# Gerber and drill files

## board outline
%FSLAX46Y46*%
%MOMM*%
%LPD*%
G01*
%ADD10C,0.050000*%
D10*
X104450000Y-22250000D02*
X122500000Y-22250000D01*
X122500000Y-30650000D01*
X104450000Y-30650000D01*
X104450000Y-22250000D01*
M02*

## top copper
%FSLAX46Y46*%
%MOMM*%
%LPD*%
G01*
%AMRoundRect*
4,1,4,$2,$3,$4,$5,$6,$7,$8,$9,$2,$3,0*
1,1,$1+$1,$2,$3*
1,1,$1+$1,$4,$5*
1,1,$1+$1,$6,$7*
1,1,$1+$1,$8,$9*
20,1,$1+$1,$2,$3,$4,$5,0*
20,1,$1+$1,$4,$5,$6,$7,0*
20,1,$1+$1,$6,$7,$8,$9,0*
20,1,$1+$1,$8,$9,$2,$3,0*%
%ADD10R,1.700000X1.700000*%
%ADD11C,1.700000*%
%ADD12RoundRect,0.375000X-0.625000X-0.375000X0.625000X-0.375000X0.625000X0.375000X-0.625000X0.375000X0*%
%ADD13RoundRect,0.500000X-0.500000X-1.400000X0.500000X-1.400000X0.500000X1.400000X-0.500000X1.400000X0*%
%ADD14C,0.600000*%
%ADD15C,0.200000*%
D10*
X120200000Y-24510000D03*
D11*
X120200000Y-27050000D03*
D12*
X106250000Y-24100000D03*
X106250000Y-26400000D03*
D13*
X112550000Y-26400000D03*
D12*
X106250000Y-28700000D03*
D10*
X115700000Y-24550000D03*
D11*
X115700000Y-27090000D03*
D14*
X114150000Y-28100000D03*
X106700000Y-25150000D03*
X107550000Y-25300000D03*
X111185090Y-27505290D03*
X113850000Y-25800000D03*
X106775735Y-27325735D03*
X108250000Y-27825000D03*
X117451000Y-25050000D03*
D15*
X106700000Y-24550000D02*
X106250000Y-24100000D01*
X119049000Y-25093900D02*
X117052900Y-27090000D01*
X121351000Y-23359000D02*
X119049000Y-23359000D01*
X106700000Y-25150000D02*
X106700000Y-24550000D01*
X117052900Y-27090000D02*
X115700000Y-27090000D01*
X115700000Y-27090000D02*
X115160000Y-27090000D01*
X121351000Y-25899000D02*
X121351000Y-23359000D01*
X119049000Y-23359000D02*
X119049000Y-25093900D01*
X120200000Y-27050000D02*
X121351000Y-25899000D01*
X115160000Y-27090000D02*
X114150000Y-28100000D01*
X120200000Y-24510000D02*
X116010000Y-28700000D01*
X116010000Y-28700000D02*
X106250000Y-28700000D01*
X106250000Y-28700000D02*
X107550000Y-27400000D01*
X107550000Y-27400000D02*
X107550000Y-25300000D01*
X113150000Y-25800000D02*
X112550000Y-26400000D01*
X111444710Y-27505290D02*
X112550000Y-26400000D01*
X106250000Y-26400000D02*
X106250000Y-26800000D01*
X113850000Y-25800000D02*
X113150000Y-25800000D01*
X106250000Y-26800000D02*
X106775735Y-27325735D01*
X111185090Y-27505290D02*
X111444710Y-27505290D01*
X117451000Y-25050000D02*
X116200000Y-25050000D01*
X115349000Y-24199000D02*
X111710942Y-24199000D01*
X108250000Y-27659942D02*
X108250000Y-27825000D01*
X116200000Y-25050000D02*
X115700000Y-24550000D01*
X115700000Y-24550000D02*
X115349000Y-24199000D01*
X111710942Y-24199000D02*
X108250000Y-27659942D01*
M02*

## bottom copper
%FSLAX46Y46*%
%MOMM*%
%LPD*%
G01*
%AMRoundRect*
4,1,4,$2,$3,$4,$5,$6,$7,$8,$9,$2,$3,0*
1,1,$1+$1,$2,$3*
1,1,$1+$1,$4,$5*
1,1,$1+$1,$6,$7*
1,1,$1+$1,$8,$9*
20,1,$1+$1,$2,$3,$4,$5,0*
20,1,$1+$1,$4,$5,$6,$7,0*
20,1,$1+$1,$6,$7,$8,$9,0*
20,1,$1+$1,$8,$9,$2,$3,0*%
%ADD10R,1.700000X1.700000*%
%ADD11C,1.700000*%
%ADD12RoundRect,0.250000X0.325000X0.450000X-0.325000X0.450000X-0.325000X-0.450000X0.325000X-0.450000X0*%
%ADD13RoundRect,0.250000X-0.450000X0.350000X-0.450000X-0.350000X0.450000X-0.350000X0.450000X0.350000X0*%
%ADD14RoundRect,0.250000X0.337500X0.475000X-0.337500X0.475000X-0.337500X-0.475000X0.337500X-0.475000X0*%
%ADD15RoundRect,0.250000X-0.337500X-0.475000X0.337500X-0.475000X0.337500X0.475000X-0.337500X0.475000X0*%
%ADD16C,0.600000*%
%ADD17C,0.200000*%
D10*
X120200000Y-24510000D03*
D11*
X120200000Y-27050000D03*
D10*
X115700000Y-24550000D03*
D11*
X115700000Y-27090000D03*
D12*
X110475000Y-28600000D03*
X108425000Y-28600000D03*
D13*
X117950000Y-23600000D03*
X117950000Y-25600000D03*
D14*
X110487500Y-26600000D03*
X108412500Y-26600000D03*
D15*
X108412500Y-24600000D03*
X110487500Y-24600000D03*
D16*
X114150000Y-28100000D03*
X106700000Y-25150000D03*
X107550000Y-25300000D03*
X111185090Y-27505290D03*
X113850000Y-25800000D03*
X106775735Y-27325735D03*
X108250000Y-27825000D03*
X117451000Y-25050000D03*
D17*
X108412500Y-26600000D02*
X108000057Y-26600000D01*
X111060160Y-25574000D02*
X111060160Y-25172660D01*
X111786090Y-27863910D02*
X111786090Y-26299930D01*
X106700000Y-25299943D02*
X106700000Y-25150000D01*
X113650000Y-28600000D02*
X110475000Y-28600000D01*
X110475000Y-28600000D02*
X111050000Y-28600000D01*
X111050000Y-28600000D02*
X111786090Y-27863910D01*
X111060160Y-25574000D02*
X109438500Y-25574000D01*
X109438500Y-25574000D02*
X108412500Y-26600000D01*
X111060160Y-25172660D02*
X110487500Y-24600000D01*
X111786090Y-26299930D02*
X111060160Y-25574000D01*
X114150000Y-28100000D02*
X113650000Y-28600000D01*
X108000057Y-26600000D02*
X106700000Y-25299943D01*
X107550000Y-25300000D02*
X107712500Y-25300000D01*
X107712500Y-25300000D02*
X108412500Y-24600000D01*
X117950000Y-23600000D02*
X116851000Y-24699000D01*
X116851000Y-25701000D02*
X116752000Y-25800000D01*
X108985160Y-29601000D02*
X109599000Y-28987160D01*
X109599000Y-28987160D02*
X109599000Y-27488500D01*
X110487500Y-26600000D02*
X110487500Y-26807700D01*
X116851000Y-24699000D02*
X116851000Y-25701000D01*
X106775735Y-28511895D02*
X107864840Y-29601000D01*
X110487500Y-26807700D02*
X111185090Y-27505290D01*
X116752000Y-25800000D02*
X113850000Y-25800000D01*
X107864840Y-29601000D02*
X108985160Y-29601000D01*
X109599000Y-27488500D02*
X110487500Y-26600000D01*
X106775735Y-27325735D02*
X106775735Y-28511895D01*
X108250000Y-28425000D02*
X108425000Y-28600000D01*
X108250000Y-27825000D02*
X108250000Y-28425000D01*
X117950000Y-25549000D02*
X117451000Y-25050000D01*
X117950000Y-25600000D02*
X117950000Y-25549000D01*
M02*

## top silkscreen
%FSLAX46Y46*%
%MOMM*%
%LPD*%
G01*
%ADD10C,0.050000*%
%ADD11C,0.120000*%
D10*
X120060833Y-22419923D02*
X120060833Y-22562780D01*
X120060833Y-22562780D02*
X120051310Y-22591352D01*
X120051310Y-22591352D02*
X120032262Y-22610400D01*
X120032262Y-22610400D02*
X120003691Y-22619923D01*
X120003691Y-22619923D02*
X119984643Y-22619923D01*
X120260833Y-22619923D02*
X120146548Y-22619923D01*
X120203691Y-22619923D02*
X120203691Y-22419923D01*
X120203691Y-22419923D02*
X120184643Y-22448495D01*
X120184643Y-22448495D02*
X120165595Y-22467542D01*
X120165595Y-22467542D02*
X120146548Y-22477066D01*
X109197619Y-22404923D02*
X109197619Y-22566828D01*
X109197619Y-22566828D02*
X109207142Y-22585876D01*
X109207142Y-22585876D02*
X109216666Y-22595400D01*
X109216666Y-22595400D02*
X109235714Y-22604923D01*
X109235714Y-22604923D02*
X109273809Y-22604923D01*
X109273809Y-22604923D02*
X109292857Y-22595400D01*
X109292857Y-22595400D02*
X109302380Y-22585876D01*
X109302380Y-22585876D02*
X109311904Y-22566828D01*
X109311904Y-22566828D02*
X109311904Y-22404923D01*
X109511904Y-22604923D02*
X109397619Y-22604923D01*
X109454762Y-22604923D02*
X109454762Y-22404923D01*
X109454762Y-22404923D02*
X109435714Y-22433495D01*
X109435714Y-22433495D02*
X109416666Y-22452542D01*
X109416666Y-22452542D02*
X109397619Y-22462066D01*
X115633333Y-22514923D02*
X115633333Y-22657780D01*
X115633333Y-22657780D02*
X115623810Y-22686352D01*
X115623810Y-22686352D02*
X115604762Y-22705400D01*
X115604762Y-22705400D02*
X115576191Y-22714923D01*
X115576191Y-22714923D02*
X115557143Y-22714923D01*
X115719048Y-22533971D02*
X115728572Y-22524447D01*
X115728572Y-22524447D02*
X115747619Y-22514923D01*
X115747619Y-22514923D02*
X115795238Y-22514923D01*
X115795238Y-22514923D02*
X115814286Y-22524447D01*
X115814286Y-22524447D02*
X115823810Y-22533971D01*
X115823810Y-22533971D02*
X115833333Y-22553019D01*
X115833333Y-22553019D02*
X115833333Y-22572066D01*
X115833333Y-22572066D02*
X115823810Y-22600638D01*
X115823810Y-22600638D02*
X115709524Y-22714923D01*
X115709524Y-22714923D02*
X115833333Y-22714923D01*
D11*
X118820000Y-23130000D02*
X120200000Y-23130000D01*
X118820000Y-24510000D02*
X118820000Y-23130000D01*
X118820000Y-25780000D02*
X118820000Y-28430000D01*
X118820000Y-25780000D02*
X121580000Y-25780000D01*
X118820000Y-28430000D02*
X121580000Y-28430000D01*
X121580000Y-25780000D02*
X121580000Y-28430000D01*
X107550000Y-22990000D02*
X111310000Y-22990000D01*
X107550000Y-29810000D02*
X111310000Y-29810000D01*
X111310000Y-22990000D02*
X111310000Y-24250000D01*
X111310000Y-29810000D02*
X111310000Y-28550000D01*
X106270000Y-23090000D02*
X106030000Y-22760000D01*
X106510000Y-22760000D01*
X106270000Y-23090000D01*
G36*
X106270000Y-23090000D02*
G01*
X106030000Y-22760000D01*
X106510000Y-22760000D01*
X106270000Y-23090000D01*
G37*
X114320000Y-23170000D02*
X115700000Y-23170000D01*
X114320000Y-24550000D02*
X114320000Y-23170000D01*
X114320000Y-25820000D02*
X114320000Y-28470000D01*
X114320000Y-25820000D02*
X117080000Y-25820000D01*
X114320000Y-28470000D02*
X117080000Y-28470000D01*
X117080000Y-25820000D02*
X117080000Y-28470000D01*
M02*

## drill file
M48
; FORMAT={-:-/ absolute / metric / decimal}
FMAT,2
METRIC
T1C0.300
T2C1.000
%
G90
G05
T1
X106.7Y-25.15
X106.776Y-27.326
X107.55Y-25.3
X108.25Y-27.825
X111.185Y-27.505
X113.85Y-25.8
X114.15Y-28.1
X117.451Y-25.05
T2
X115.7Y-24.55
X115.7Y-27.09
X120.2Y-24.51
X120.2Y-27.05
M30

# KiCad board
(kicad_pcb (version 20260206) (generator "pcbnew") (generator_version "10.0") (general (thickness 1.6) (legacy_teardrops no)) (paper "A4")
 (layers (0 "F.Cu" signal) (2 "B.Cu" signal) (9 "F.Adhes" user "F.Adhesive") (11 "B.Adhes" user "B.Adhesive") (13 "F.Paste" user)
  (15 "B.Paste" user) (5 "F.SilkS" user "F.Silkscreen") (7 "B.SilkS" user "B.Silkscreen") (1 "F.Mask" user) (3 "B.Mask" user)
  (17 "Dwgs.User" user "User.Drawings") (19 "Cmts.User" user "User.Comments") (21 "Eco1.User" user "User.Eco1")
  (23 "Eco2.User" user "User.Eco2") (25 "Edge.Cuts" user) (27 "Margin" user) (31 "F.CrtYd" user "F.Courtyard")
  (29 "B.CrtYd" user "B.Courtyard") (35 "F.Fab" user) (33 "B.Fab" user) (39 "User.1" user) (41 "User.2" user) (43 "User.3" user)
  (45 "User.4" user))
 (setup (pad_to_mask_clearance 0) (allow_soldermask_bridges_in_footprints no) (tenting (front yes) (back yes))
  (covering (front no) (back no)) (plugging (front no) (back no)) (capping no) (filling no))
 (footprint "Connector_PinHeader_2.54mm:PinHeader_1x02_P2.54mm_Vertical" (layer "F.Cu") (at 120.2 24.51)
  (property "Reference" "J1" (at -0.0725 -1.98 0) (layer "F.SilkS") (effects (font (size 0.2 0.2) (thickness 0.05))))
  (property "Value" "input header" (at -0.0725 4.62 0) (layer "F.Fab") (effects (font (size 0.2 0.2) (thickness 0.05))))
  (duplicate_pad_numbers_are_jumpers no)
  (fp_line (start -1.38 -1.38) (end 0 -1.38) (stroke (width 0.12) (type solid)) (layer "F.SilkS"))
  (fp_line (start -1.38 0) (end -1.38 -1.38) (stroke (width 0.12) (type solid)) (layer "F.SilkS"))
  (fp_line (start -1.38 1.27) (end -1.38 3.92) (stroke (width 0.12) (type solid)) (layer "F.SilkS"))
  (fp_line (start -1.38 1.27) (end 1.38 1.27) (stroke (width 0.12) (type solid)) (layer "F.SilkS"))
  (fp_line (start -1.38 3.92) (end 1.38 3.92) (stroke (width 0.12) (type solid)) (layer "F.SilkS"))
  (fp_line (start 1.38 1.27) (end 1.38 3.92) (stroke (width 0.12) (type solid)) (layer "F.SilkS"))
  (pad "1" thru_hole rect (at 0 0) (size 1.7 1.7) (drill 1) (layers "*.Cu" "*.Mask") (remove_unused_layers no) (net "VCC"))
  (pad "2" thru_hole circle (at 0 2.54) (size 1.7 1.7) (drill 1) (layers "*.Cu" "*.Mask") (remove_unused_layers no) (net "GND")))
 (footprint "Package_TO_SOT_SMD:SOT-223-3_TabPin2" (layer "F.Cu") (at 109.4 26.4)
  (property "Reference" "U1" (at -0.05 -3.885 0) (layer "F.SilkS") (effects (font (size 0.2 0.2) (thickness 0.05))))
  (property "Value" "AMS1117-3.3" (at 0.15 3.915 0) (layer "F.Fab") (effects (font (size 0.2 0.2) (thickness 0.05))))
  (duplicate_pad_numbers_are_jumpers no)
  (fp_line (start -1.85 -3.41) (end 1.91 -3.41) (stroke (width 0.12) (type solid)) (layer "F.SilkS"))
  (fp_line (start -1.85 3.41) (end 1.91 3.41) (stroke (width 0.12) (type solid)) (layer "F.SilkS"))
  (fp_line (start 1.91 -3.41) (end 1.91 -2.15) (stroke (width 0.12) (type solid)) (layer "F.SilkS"))
  (fp_line (start 1.91 3.41) (end 1.91 2.15) (stroke (width 0.12) (type solid)) (layer "F.SilkS"))
  (fp_poly
   (pts (xy -3.13 -3.31) (xy -3.37 -3.64) (xy -2.89 -3.64) (xy -3.13 -3.31)) (stroke (width 0.12) (type solid)) (fill yes) (layer "F.SilkS"))
  (pad "1" smd roundrect (at -3.15 -2.3) (size 2 1.5) (layers "F.Cu" "F.Mask" "F.Paste") (roundrect_rratio 0.25) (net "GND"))
  (pad "2" smd roundrect (at -3.15 0) (size 2 1.5) (layers "F.Cu" "F.Mask" "F.Paste") (roundrect_rratio 0.25) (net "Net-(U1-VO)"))
  (pad "2" smd roundrect (at 3.15 0) (size 2 3.8) (layers "F.Cu" "F.Mask" "F.Paste") (roundrect_rratio 0.25) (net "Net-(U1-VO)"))
  (pad "3" smd roundrect (at -3.15 2.3) (size 2 1.5) (layers "F.Cu" "F.Mask" "F.Paste") (roundrect_rratio 0.25) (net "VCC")))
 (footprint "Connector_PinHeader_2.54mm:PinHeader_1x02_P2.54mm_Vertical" (layer "F.Cu") (at 115.7 24.55)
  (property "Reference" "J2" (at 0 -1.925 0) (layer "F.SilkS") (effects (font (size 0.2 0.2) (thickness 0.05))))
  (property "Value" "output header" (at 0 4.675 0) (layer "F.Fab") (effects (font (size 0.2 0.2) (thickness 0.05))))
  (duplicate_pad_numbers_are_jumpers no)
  (fp_line (start -1.38 -1.38) (end 0 -1.38) (stroke (width 0.12) (type solid)) (layer "F.SilkS"))
  (fp_line (start -1.38 0) (end -1.38 -1.38) (stroke (width 0.12) (type solid)) (layer "F.SilkS"))
  (fp_line (start -1.38 1.27) (end -1.38 3.92) (stroke (width 0.12) (type solid)) (layer "F.SilkS"))
  (fp_line (start -1.38 1.27) (end 1.38 1.27) (stroke (width 0.12) (type solid)) (layer "F.SilkS"))
  (fp_line (start -1.38 3.92) (end 1.38 3.92) (stroke (width 0.12) (type solid)) (layer "F.SilkS"))
  (fp_line (start 1.38 1.27) (end 1.38 3.92) (stroke (width 0.12) (type solid)) (layer "F.SilkS"))
  (pad "1" thru_hole rect (at 0 0) (size 1.7 1.7) (drill 1) (layers "*.Cu" "*.Mask") (remove_unused_layers no) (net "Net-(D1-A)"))
  (pad "2" thru_hole circle (at 0 2.54) (size 1.7 1.7) (drill 1) (layers "*.Cu" "*.Mask") (remove_unused_layers no) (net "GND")))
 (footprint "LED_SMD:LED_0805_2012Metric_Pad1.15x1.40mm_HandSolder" (layer "B.Cu") (at 109.45 28.6 180)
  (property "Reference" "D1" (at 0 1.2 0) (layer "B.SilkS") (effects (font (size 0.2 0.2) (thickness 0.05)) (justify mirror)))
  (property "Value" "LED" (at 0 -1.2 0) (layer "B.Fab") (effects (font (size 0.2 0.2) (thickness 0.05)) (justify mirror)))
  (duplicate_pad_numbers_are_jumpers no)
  (pad "1" smd roundrect (at -1.025 0 180) (size 1.15 1.4) (layers "B.Cu" "B.Mask" "B.Paste") (roundrect_rratio 0.217391) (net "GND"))
  (pad "2" smd roundrect (at 1.025 0 180) (size 1.15 1.4) (layers "B.Cu" "B.Mask" "B.Paste") (roundrect_rratio 0.217391) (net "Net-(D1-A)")))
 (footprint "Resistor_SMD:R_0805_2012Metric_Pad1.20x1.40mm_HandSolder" (layer "B.Cu") (at 117.95 24.6 -90)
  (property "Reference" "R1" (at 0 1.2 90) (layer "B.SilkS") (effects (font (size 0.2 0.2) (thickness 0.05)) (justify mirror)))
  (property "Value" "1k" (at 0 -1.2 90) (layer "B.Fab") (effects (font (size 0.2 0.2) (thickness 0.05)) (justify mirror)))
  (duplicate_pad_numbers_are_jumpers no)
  (pad "1" smd roundrect (at -1 0 270) (size 1.2 1.4) (layers "B.Cu" "B.Mask" "B.Paste") (roundrect_rratio 0.208333) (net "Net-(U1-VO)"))
  (pad "2" smd roundrect (at 1 0 270) (size 1.2 1.4) (layers "B.Cu" "B.Mask" "B.Paste") (roundrect_rratio 0.208333) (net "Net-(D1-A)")))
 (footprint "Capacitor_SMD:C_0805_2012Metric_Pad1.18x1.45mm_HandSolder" (layer "B.Cu") (at 109.45 26.6 180)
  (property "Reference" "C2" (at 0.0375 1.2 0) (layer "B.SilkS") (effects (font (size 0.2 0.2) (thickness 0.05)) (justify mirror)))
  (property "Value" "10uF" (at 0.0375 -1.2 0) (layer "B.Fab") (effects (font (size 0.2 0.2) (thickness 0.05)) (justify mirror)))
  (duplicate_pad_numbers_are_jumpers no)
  (pad "1" smd roundrect (at -1.0375 0 180) (size 1.175 1.45) (layers "B.Cu" "B.Mask" "B.Paste") (roundrect_rratio 0.212766)
   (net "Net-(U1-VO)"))
  (pad "2" smd roundrect (at 1.0375 0 180) (size 1.175 1.45) (layers "B.Cu" "B.Mask" "B.Paste") (roundrect_rratio 0.212766) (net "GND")))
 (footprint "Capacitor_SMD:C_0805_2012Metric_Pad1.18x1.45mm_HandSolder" (layer "B.Cu") (at 109.45 24.6)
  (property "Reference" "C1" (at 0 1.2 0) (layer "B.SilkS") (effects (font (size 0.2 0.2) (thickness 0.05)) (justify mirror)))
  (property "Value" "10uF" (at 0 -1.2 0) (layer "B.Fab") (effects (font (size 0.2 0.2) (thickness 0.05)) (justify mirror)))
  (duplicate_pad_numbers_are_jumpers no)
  (pad "1" smd roundrect (at -1.0375 0) (size 1.175 1.45) (layers "B.Cu" "B.Mask" "B.Paste") (roundrect_rratio 0.212766) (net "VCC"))
  (pad "2" smd roundrect (at 1.0375 0) (size 1.175 1.45) (layers "B.Cu" "B.Mask" "B.Paste") (roundrect_rratio 0.212766) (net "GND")))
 (gr_rect (start 104.45 22.25) (end 122.5 30.65) (stroke (width 0.05) (type default)) (fill no) (layer "Edge.Cuts"))
 (segment (start 106.7 24.55) (end 106.25 24.1) (width 0.2) (layer "F.Cu") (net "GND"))
 (segment (start 119.049 25.0939) (end 117.0529 27.09) (width 0.2) (layer "F.Cu") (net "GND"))
 (segment (start 121.351 23.359) (end 119.049 23.359) (width 0.2) (layer "F.Cu") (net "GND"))
 (segment (start 106.7 25.15) (end 106.7 24.55) (width 0.2) (layer "F.Cu") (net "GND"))
 (segment (start 117.0529 27.09) (end 115.7 27.09) (width 0.2) (layer "F.Cu") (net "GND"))
 (segment (start 115.7 27.09) (end 115.16 27.09) (width 0.2) (layer "F.Cu") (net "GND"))
 (segment (start 121.351 25.899) (end 121.351 23.359) (width 0.2) (layer "F.Cu") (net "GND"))
 (segment (start 119.049 23.359) (end 119.049 25.0939) (width 0.2) (layer "F.Cu") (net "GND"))
 (segment (start 120.2 27.05) (end 121.351 25.899) (width 0.2) (layer "F.Cu") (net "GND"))
 (segment (start 115.16 27.09) (end 114.15 28.1) (width 0.2) (layer "F.Cu") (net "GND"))
 (via (at 114.15 28.1) (size 0.6) (drill 0.3) (layers "F.Cu" "B.Cu") (capping no) (covering (front no) (back no))
  (plugging (front no) (back no)) (filling no) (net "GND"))
 (via (at 106.7 25.15) (size 0.6) (drill 0.3) (layers "F.Cu" "B.Cu") (capping no) (covering (front no) (back no))
  (plugging (front no) (back no)) (filling no) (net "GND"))
 (segment (start 108.4125 26.6) (end 108.000057 26.6) (width 0.2) (layer "B.Cu") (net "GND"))
 (segment (start 111.06016 25.574) (end 111.06016 25.17266) (width 0.2) (layer "B.Cu") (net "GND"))
 (segment (start 111.78609 27.86391) (end 111.78609 26.29993) (width 0.2) (layer "B.Cu") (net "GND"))
 (segment (start 106.7 25.299943) (end 106.7 25.15) (width 0.2) (layer "B.Cu") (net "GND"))
 (segment (start 113.65 28.6) (end 110.475 28.6) (width 0.2) (layer "B.Cu") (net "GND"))
 (segment (start 110.475 28.6) (end 111.05 28.6) (width 0.2) (layer "B.Cu") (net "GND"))
 (segment (start 111.05 28.6) (end 111.78609 27.86391) (width 0.2) (layer "B.Cu") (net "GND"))
 (segment (start 111.06016 25.574) (end 109.4385 25.574) (width 0.2) (layer "B.Cu") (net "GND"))
 (segment (start 109.4385 25.574) (end 108.4125 26.6) (width 0.2) (layer "B.Cu") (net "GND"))
 (segment (start 111.06016 25.17266) (end 110.4875 24.6) (width 0.2) (layer "B.Cu") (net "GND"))
 (segment (start 111.78609 26.29993) (end 111.06016 25.574) (width 0.2) (layer "B.Cu") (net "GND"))
 (segment (start 114.15 28.1) (end 113.65 28.6) (width 0.2) (layer "B.Cu") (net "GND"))
 (segment (start 108.000057 26.6) (end 106.7 25.299943) (width 0.2) (layer "B.Cu") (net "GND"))
 (segment (start 120.2 24.51) (end 116.01 28.7) (width 0.2) (layer "F.Cu") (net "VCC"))
 (segment (start 116.01 28.7) (end 106.25 28.7) (width 0.2) (layer "F.Cu") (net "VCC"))
 (segment (start 106.25 28.7) (end 107.55 27.4) (width 0.2) (layer "F.Cu") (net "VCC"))
 (segment (start 107.55 27.4) (end 107.55 25.3) (width 0.2) (layer "F.Cu") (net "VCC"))
 (via (at 107.55 25.3) (size 0.6) (drill 0.3) (layers "F.Cu" "B.Cu") (capping no) (covering (front no) (back no))
  (plugging (front no) (back no)) (filling no) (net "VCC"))
 (segment (start 107.55 25.3) (end 107.7125 25.3) (width 0.2) (layer "B.Cu") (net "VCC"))
 (segment (start 107.7125 25.3) (end 108.4125 24.6) (width 0.2) (layer "B.Cu") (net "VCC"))
 (segment (start 113.15 25.8) (end 112.55 26.4) (width 0.2) (layer "F.Cu") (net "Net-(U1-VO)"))
 (segment (start 111.44471 27.50529) (end 112.55 26.4) (width 0.2) (layer "F.Cu") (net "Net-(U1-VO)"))
 (segment (start 106.25 26.4) (end 106.25 26.8) (width 0.2) (layer "F.Cu") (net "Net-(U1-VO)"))
 (segment (start 113.85 25.8) (end 113.15 25.8) (width 0.2) (layer "F.Cu") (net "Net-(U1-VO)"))
 (segment (start 106.25 26.8) (end 106.775735 27.325735) (width 0.2) (layer "F.Cu") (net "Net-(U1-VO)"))
 (segment (start 111.18509 27.50529) (end 111.44471 27.50529) (width 0.2) (layer "F.Cu") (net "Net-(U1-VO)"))
 (via (at 111.18509 27.50529) (size 0.6) (drill 0.3) (layers "F.Cu" "B.Cu") (capping no) (covering (front no) (back no))
  (plugging (front no) (back no)) (filling no) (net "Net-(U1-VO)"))
 (via (at 113.85 25.8) (size 0.6) (drill 0.3) (layers "F.Cu" "B.Cu") (capping no) (covering (front no) (back no))
  (plugging (front no) (back no)) (filling no) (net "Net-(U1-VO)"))
 (via (at 106.775735 27.325735) (size 0.6) (drill 0.3) (layers "F.Cu" "B.Cu") (capping no) (covering (front no) (back no))
  (plugging (front no) (back no)) (filling no) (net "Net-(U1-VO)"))
 (segment (start 117.95 23.6) (end 116.851 24.699) (width 0.2) (layer "B.Cu") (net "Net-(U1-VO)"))
 (segment (start 116.851 25.701) (end 116.752 25.8) (width 0.2) (layer "B.Cu") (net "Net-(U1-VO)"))
 (segment (start 108.98516 29.601) (end 109.599 28.98716) (width 0.2) (layer "B.Cu") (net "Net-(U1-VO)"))
 (segment (start 109.599 28.98716) (end 109.599 27.4885) (width 0.2) (layer "B.Cu") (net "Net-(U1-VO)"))
 (segment (start 110.4875 26.6) (end 110.4875 26.8077) (width 0.2) (layer "B.Cu") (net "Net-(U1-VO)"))
 (segment (start 116.851 24.699) (end 116.851 25.701) (width 0.2) (layer "B.Cu") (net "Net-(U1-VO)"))
 (segment (start 106.775735 28.511895) (end 107.86484 29.601) (width 0.2) (layer "B.Cu") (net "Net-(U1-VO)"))
 (segment (start 110.4875 26.8077) (end 111.18509 27.50529) (width 0.2) (layer "B.Cu") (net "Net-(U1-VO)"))
 (segment (start 116.752 25.8) (end 113.85 25.8) (width 0.2) (layer "B.Cu") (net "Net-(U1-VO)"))
 (segment (start 107.86484 29.601) (end 108.98516 29.601) (width 0.2) (layer "B.Cu") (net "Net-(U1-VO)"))
 (segment (start 109.599 27.4885) (end 110.4875 26.6) (width 0.2) (layer "B.Cu") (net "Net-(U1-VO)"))
 (segment (start 106.775735 27.325735) (end 106.775735 28.511895) (width 0.2) (layer "B.Cu") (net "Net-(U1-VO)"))
 (segment (start 117.451 25.05) (end 116.2 25.05) (width 0.2) (layer "F.Cu") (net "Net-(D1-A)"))
 (segment (start 115.349 24.199) (end 111.710942 24.199) (width 0.2) (layer "F.Cu") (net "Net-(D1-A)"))
 (segment (start 108.25 27.659942) (end 108.25 27.825) (width 0.2) (layer "F.Cu") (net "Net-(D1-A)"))
 (segment (start 116.2 25.05) (end 115.7 24.55) (width 0.2) (layer "F.Cu") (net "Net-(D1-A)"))
 (segment (start 115.7 24.55) (end 115.349 24.199) (width 0.2) (layer "F.Cu") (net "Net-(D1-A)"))
 (segment (start 111.710942 24.199) (end 108.25 27.659942) (width 0.2) (layer "F.Cu") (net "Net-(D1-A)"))
 (via (at 108.25 27.825) (size 0.6) (drill 0.3) (layers "F.Cu" "B.Cu") (capping no) (covering (front no) (back no))
  (plugging (front no) (back no)) (filling no) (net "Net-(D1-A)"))
 (via (at 117.451 25.05) (size 0.6) (drill 0.3) (layers "F.Cu" "B.Cu") (capping no) (covering (front no) (back no))
  (plugging (front no) (back no)) (filling no) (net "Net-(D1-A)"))
 (segment (start 108.25 28.425) (end 108.425 28.6) (width 0.2) (layer "B.Cu") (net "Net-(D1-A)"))
 (segment (start 108.25 27.825) (end 108.25 28.425) (width 0.2) (layer "B.Cu") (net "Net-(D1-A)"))
 (segment (start 117.95 25.549) (end 117.451 25.05) (width 0.2) (layer "B.Cu") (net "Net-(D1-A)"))
 (segment (start 117.95 25.6) (end 117.95 25.549) (width 0.2) (layer "B.Cu") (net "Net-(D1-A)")))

